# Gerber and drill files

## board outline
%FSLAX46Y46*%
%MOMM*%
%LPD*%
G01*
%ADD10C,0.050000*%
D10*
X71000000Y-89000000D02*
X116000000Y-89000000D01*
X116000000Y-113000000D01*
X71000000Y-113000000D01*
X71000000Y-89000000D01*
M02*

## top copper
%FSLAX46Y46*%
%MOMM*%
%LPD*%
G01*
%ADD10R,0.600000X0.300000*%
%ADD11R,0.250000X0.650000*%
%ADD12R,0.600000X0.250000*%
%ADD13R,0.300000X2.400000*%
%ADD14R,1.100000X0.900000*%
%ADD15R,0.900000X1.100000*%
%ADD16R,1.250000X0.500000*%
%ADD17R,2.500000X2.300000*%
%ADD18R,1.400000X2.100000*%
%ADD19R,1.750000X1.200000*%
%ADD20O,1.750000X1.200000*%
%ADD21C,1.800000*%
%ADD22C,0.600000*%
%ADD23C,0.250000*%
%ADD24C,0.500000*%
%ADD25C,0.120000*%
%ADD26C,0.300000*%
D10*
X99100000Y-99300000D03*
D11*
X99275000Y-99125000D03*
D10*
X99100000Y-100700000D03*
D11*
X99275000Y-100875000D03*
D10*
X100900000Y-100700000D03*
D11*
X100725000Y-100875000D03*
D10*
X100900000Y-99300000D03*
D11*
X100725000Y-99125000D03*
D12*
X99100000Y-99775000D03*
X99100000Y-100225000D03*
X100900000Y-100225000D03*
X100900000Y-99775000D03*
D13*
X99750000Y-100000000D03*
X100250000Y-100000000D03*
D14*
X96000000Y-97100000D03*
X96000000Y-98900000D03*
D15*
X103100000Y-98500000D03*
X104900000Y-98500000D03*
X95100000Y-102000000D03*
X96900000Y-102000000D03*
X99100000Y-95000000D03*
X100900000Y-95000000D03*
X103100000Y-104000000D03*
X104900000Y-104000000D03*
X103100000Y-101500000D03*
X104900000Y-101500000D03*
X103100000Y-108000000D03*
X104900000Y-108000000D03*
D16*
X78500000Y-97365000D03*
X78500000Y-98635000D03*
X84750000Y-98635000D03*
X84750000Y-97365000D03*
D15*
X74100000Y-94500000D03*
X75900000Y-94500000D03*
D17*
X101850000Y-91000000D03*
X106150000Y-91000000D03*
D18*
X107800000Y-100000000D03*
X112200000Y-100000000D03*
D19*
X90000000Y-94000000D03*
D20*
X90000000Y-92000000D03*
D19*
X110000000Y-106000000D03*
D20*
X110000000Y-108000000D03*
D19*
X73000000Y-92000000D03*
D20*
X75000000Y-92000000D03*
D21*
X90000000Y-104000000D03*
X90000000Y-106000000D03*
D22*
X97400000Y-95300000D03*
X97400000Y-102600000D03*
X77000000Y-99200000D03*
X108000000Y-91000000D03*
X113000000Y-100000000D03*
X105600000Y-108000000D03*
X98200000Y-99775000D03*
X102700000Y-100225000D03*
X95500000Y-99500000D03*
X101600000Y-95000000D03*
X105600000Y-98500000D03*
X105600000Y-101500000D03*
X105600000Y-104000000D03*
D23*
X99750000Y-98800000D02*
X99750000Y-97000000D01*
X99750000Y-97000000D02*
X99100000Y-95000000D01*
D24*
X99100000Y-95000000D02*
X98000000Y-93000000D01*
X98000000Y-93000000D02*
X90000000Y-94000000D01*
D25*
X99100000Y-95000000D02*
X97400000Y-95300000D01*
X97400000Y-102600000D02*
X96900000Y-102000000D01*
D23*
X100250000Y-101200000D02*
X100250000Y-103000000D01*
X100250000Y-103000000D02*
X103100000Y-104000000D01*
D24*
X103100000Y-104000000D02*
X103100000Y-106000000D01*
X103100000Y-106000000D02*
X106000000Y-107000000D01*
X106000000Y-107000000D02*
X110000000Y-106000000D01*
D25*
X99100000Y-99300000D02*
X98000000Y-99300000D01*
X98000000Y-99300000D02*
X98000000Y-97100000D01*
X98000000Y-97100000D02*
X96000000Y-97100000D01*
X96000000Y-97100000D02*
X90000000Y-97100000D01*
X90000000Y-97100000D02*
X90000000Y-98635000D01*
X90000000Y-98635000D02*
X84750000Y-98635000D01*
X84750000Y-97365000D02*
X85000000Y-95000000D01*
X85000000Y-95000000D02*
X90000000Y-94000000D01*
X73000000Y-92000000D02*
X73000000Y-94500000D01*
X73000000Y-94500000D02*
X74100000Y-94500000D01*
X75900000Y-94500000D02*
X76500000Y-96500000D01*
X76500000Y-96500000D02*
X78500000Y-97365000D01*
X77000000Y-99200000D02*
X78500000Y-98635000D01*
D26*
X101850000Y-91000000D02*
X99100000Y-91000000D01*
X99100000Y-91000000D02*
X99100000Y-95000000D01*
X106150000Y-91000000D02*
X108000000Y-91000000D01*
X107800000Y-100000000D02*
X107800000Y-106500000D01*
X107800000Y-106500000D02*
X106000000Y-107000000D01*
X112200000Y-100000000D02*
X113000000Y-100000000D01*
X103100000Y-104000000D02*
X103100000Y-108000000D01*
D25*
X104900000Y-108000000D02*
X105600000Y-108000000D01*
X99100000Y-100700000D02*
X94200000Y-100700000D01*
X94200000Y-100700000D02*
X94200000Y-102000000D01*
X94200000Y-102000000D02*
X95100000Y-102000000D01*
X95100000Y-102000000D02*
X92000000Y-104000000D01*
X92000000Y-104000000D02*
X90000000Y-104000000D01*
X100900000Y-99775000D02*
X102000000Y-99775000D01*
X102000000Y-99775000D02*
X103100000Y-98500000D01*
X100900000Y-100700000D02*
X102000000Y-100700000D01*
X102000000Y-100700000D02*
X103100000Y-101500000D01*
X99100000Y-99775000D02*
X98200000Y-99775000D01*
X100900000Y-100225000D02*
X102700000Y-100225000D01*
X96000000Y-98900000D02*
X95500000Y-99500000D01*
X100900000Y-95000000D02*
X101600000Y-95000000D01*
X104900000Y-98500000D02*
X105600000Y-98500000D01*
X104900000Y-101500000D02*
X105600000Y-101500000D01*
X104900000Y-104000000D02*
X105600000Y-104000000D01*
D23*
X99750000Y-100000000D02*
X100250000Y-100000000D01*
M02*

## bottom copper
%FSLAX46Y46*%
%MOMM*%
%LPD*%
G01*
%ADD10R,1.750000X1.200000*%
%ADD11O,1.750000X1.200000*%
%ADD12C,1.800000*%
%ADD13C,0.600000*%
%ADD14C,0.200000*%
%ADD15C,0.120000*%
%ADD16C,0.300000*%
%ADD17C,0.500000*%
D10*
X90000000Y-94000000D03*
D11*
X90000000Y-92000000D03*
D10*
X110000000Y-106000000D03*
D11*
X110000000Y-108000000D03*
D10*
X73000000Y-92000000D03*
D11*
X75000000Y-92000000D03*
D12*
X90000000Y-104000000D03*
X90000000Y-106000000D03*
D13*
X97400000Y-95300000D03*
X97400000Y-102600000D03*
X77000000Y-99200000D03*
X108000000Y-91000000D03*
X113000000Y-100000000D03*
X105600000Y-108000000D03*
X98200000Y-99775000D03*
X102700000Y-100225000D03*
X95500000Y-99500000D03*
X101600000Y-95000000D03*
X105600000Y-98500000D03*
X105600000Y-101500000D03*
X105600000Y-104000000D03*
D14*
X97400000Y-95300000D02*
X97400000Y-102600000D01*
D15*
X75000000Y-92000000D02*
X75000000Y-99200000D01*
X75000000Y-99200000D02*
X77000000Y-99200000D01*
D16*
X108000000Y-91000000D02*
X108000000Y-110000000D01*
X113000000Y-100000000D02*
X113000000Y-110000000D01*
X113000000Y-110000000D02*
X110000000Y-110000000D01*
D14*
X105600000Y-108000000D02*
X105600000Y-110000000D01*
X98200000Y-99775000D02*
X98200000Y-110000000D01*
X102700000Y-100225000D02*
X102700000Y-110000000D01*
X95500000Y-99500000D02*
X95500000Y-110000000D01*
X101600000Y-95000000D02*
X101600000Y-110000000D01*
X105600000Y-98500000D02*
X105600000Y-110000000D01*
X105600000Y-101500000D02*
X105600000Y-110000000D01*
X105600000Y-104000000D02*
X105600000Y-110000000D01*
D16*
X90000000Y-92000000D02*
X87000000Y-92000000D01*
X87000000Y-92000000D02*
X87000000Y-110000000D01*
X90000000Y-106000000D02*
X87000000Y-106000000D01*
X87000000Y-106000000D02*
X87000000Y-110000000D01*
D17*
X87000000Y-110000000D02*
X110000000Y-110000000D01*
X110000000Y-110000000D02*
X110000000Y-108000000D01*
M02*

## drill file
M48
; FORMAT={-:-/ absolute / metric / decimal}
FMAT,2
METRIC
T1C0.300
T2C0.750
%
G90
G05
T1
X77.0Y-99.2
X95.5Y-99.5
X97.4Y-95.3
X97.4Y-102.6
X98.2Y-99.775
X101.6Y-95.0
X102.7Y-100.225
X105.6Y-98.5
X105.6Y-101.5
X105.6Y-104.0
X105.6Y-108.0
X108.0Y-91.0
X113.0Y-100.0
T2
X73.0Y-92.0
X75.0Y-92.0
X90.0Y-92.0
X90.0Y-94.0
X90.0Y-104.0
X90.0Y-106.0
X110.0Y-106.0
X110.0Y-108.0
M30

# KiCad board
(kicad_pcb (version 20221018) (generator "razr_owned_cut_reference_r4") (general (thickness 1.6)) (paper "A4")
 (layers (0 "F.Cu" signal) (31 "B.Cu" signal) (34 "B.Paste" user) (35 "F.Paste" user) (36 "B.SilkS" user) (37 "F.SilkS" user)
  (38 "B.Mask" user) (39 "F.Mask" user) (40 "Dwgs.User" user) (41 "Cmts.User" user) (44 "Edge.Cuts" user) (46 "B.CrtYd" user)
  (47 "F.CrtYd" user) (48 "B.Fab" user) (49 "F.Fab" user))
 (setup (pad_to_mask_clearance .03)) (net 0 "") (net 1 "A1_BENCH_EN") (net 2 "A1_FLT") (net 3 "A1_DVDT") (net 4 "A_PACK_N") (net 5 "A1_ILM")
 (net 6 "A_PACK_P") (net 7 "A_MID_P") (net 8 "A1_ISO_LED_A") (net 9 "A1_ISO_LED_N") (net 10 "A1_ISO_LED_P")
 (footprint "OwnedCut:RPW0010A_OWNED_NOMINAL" (layer "F.Cu") (at 100 100)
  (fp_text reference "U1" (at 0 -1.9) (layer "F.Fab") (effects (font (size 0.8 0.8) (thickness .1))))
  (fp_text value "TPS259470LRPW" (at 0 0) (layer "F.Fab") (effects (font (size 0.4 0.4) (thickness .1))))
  (pad "1" smd rect (at -0.9 -0.7) (size 0.6 0.3) (layers "F.Cu" "F.Paste" "F.Mask") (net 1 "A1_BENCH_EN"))
  (pad "1" smd rect (at -0.725 -0.875) (size 0.25 0.65) (layers "F.Cu" "F.Paste" "F.Mask") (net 1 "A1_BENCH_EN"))
  (pad "4" smd rect (at -0.9 0.7) (size 0.6 0.3) (layers "F.Cu" "F.Paste" "F.Mask") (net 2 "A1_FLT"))
  (pad "4" smd rect (at -0.725 0.875) (size 0.25 0.65) (layers "F.Cu" "F.Paste" "F.Mask") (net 2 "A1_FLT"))
  (pad "7" smd rect (at 0.9 0.7) (size 0.6 0.3) (layers "F.Cu" "F.Paste" "F.Mask") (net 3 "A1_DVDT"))
  (pad "7" smd rect (at 0.725 0.875) (size 0.25 0.65) (layers "F.Cu" "F.Paste" "F.Mask") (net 3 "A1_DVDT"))
  (pad "10" smd rect (at 0.9 -0.7) (size 0.6 0.3) (layers "F.Cu" "F.Paste" "F.Mask"))
  (pad "10" smd rect (at 0.725 -0.875) (size 0.25 0.65) (layers "F.Cu" "F.Paste" "F.Mask"))
  (pad "2" smd rect (at -0.9 -0.225) (size 0.6 0.25) (layers "F.Cu" "F.Paste" "F.Mask") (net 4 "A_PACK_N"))
  (pad "3" smd rect (at -0.9 0.225) (size 0.6 0.25) (layers "F.Cu" "F.Paste" "F.Mask"))
  (pad "8" smd rect (at 0.9 0.225) (size 0.6 0.25) (layers "F.Cu" "F.Paste" "F.Mask") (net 4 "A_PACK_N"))
  (pad "9" smd rect (at 0.9 -0.225) (size 0.6 0.25) (layers "F.Cu" "F.Paste" "F.Mask") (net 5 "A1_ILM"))
  (pad "5" smd rect (at -0.25 0) (size 0.3 2.4) (layers "F.Cu" "F.Paste" "F.Mask") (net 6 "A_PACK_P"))
  (pad "6" smd rect (at 0.25 0) (size 0.3 2.4) (layers "F.Cu" "F.Paste" "F.Mask") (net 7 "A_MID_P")))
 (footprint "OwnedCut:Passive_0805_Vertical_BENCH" (layer "F.Cu") (at 96 98)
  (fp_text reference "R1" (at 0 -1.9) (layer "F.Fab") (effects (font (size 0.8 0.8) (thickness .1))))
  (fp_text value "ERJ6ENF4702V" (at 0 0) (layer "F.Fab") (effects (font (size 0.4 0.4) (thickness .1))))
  (pad "1" smd rect (at 0 -0.9) (size 1.1 0.9) (layers "F.Cu" "F.Paste" "F.Mask") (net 1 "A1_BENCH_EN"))
  (pad "2" smd rect (at 0 0.9) (size 1.1 0.9) (layers "F.Cu" "F.Paste" "F.Mask") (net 4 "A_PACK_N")))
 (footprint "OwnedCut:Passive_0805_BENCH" (layer "F.Cu") (at 104 98.5)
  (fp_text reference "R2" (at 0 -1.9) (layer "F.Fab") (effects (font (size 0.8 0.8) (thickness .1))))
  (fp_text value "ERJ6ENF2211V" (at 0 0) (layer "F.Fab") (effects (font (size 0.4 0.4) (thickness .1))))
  (pad "1" smd rect (at -0.9 0) (size 0.9 1.1) (layers "F.Cu" "F.Paste" "F.Mask") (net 5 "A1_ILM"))
  (pad "2" smd rect (at 0.9 0) (size 0.9 1.1) (layers "F.Cu" "F.Paste" "F.Mask") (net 4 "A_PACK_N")))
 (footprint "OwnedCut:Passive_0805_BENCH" (layer "F.Cu") (at 96 102)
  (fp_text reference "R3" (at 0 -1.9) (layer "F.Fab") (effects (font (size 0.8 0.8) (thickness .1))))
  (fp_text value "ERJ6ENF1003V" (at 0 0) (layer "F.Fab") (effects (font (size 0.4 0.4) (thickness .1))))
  (pad "1" smd rect (at -0.9 0) (size 0.9 1.1) (layers "F.Cu" "F.Paste" "F.Mask") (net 2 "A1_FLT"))
  (pad "2" smd rect (at 0.9 0) (size 0.9 1.1) (layers "F.Cu" "F.Paste" "F.Mask") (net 6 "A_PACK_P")))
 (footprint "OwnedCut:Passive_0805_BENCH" (layer "F.Cu") (at 100 95)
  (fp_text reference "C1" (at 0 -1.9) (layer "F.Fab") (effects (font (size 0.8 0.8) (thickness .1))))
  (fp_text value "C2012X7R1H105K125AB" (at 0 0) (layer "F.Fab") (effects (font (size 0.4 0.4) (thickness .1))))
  (pad "1" smd rect (at -0.9 0) (size 0.9 1.1) (layers "F.Cu" "F.Paste" "F.Mask") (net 6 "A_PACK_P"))
  (pad "2" smd rect (at 0.9 0) (size 0.9 1.1) (layers "F.Cu" "F.Paste" "F.Mask") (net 4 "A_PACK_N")))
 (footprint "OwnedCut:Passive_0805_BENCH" (layer "F.Cu") (at 104 104)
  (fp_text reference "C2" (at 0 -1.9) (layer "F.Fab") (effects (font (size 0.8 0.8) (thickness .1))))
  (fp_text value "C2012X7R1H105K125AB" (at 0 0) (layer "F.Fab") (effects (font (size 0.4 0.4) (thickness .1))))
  (pad "1" smd rect (at -0.9 0) (size 0.9 1.1) (layers "F.Cu" "F.Paste" "F.Mask") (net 7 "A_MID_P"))
  (pad "2" smd rect (at 0.9 0) (size 0.9 1.1) (layers "F.Cu" "F.Paste" "F.Mask") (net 4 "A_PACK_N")))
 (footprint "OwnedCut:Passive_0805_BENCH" (layer "F.Cu") (at 104 101.5)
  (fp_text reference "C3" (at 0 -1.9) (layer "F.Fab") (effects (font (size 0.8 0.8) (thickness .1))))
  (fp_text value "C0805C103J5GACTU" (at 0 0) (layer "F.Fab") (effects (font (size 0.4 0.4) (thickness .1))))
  (pad "1" smd rect (at -0.9 0) (size 0.9 1.1) (layers "F.Cu" "F.Paste" "F.Mask") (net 3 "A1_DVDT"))
  (pad "2" smd rect (at 0.9 0) (size 0.9 1.1) (layers "F.Cu" "F.Paste" "F.Mask") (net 4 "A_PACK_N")))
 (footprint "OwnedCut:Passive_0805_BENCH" (layer "F.Cu") (at 104 108)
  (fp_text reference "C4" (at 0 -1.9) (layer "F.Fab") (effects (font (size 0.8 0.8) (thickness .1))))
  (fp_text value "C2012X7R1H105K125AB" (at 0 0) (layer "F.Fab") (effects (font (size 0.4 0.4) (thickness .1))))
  (pad "1" smd rect (at -0.9 0) (size 0.9 1.1) (layers "F.Cu" "F.Paste" "F.Mask") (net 7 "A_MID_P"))
  (pad "2" smd rect (at 0.9 0) (size 0.9 1.1) (layers "F.Cu" "F.Paste" "F.Mask") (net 4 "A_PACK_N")))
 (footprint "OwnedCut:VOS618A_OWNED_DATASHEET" (layer "F.Cu") (at 81.625 98)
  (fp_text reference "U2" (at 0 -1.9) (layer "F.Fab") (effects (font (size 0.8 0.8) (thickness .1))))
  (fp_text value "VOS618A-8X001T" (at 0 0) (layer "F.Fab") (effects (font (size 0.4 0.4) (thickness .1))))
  (pad "1" smd rect (at -3.125 -0.635) (size 1.25 0.5) (layers "F.Cu" "F.Paste" "F.Mask") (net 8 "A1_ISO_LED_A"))
  (pad "2" smd rect (at -3.125 0.635) (size 1.25 0.5) (layers "F.Cu" "F.Paste" "F.Mask") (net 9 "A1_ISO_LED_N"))
  (pad "3" smd rect (at 3.125 0.635) (size 1.25 0.5) (layers "F.Cu" "F.Paste" "F.Mask") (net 1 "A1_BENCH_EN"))
  (pad "4" smd rect (at 3.125 -0.635) (size 1.25 0.5) (layers "F.Cu" "F.Paste" "F.Mask") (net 6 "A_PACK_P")))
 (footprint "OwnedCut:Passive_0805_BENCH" (layer "F.Cu") (at 75 94.5)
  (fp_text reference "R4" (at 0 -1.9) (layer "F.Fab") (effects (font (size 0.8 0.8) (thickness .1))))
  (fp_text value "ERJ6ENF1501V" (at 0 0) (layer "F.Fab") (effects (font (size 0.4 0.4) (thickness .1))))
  (pad "1" smd rect (at -0.9 0) (size 0.9 1.1) (layers "F.Cu" "F.Paste" "F.Mask") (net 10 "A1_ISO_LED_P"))
  (pad "2" smd rect (at 0.9 0) (size 0.9 1.1) (layers "F.Cu" "F.Paste" "F.Mask") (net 8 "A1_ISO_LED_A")))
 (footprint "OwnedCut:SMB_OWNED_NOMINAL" (layer "F.Cu") (at 104 91)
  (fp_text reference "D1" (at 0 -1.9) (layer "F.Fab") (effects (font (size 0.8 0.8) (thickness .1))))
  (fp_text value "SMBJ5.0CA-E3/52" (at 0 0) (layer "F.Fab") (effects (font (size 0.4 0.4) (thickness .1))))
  (pad "1" smd rect (at -2.15 0) (size 2.5 2.3) (layers "F.Cu" "F.Paste" "F.Mask") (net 6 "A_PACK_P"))
  (pad "2" smd rect (at 2.15 0) (size 2.5 2.3) (layers "F.Cu" "F.Paste" "F.Mask") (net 4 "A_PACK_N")))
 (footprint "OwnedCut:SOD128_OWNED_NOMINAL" (layer "F.Cu") (at 110 100)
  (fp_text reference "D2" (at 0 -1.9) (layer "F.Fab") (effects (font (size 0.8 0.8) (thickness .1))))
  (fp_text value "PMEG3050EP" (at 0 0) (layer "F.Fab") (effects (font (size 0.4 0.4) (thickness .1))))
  (pad "1" smd rect (at -2.2 0) (size 1.4 2.1) (layers "F.Cu" "F.Paste" "F.Mask") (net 7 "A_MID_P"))
  (pad "2" smd rect (at 2.2 0) (size 1.4 2.1) (layers "F.Cu" "F.Paste" "F.Mask") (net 4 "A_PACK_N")))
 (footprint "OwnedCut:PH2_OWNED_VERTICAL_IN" (layer "F.Cu") (at 90 94)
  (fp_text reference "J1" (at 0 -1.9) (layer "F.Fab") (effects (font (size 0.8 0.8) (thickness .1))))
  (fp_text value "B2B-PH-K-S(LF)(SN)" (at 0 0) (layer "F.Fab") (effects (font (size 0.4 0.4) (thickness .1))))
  (pad "1" thru_hole rect (at 0 0) (size 1.75 1.2) (drill .75) (layers "*.Cu" "*.Mask") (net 6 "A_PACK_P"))
  (pad "2" thru_hole oval (at 0 -2) (size 1.75 1.2) (drill .75) (layers "*.Cu" "*.Mask") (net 4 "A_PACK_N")))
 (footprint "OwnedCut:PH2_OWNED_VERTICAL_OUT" (layer "F.Cu") (at 110 106)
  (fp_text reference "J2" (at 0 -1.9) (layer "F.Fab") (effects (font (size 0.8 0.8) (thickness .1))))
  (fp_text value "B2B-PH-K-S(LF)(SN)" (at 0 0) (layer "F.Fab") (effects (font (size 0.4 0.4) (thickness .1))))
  (pad "1" thru_hole rect (at 0 0) (size 1.75 1.2) (drill .75) (layers "*.Cu" "*.Mask") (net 7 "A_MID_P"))
  (pad "2" thru_hole oval (at 0 2) (size 1.75 1.2) (drill .75) (layers "*.Cu" "*.Mask") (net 4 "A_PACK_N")))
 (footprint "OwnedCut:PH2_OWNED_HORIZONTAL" (layer "F.Cu") (at 73 92)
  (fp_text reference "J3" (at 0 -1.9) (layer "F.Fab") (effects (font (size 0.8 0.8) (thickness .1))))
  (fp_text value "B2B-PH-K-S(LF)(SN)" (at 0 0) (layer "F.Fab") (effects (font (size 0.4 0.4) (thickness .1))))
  (pad "1" thru_hole rect (at 0 0) (size 1.75 1.2) (drill .75) (layers "*.Cu" "*.Mask") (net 10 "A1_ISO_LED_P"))
  (pad "2" thru_hole oval (at 2 0) (size 1.75 1.2) (drill .75) (layers "*.Cu" "*.Mask") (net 9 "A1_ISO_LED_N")))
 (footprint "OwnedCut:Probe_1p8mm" (layer "F.Cu") (at 90 104)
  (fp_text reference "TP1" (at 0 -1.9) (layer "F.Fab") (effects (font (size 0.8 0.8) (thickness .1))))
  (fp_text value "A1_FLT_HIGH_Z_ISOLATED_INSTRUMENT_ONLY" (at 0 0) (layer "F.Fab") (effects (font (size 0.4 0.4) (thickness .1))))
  (pad "1" thru_hole circle (at 0 0) (size 1.8 1.8) (drill .75) (layers "*.Cu" "*.Mask") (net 2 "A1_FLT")))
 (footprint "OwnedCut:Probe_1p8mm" (layer "F.Cu") (at 90 106)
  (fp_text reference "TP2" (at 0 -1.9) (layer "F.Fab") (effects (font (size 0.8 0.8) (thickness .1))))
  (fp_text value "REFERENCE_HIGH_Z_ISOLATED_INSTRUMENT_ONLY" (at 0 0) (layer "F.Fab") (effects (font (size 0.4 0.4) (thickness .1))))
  (pad "1" thru_hole circle (at 0 0) (size 1.8 1.8) (drill .75) (layers "*.Cu" "*.Mask") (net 4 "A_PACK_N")))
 (segment (start 99.75 98.8) (end 99.75 97) (width 0.25) (layer "F.Cu") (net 6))
 (segment (start 99.75 97) (end 99.1 95) (width 0.25) (layer "F.Cu") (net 6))
 (segment (start 99.1 95) (end 98 93) (width 0.5) (layer "F.Cu") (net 6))
 (segment (start 98 93) (end 90 94) (width 0.5) (layer "F.Cu") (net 6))
 (segment (start 99.1 95) (end 97.4 95.3) (width 0.12) (layer "F.Cu") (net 6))
 (via (at 97.4 95.3) (size .6) (drill .3) (layers "F.Cu" "B.Cu") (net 6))
 (segment (start 97.4 95.3) (end 97.4 102.6) (width 0.2) (layer "B.Cu") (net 6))
 (via (at 97.4 102.6) (size .6) (drill .3) (layers "F.Cu" "B.Cu") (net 6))
 (segment (start 97.4 102.6) (end 96.9 102) (width 0.12) (layer "F.Cu") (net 6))
 (segment (start 100.25 101.2) (end 100.25 103) (width 0.25) (layer "F.Cu") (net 7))
 (segment (start 100.25 103) (end 103.1 104) (width 0.25) (layer "F.Cu") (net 7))
 (segment (start 103.1 104) (end 103.1 106) (width 0.5) (layer "F.Cu") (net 7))
 (segment (start 103.1 106) (end 106 107) (width 0.5) (layer "F.Cu") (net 7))
 (segment (start 106 107) (end 110 106) (width 0.5) (layer "F.Cu") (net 7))
 (segment (start 99.1 99.3) (end 98 99.3) (width 0.12) (layer "F.Cu") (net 1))
 (segment (start 98 99.3) (end 98 97.1) (width 0.12) (layer "F.Cu") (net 1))
 (segment (start 98 97.1) (end 96 97.1) (width 0.12) (layer "F.Cu") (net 1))
 (segment (start 96 97.1) (end 90 97.1) (width 0.12) (layer "F.Cu") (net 1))
 (segment (start 90 97.1) (end 90 98.635) (width 0.12) (layer "F.Cu") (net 1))
 (segment (start 90 98.635) (end 84.75 98.635) (width 0.12) (layer "F.Cu") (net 1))
 (segment (start 84.75 97.365) (end 85 95) (width 0.12) (layer "F.Cu") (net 6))
 (segment (start 85 95) (end 90 94) (width 0.12) (layer "F.Cu") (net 6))
 (segment (start 73 92) (end 73 94.5) (width 0.12) (layer "F.Cu") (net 10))
 (segment (start 73 94.5) (end 74.1 94.5) (width 0.12) (layer "F.Cu") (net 10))
 (segment (start 75.9 94.5) (end 76.5 96.5) (width 0.12) (layer "F.Cu") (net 8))
 (segment (start 76.5 96.5) (end 78.5 97.365) (width 0.12) (layer "F.Cu") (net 8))
 (segment (start 75 92) (end 75 99.2) (width 0.12) (layer "B.Cu") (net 9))
 (segment (start 75 99.2) (end 77 99.2) (width 0.12) (layer "B.Cu") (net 9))
 (via (at 77 99.2) (size .6) (drill .3) (layers "F.Cu" "B.Cu") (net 9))
 (segment (start 77 99.2) (end 78.5 98.635) (width 0.12) (layer "F.Cu") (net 9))
 (segment (start 101.85 91) (end 99.1 91) (width 0.3) (layer "F.Cu") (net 6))
 (segment (start 99.1 91) (end 99.1 95) (width 0.3) (layer "F.Cu") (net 6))
 (segment (start 106.15 91) (end 108 91) (width 0.3) (layer "F.Cu") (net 4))
 (via (at 108 91) (size .6) (drill .3) (layers "F.Cu" "B.Cu") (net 4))
 (segment (start 108 91) (end 108 110) (width 0.3) (layer "B.Cu") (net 4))
 (segment (start 107.8 100) (end 107.8 106.5) (width 0.3) (layer "F.Cu") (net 7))
 (segment (start 107.8 106.5) (end 106 107) (width 0.3) (layer "F.Cu") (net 7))
 (segment (start 112.2 100) (end 113 100) (width 0.3) (layer "F.Cu") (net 4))
 (via (at 113 100) (size .6) (drill .3) (layers "F.Cu" "B.Cu") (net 4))
 (segment (start 113 100) (end 113 110) (width 0.3) (layer "B.Cu") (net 4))
 (segment (start 113 110) (end 110 110) (width 0.3) (layer "B.Cu") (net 4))
 (segment (start 103.1 104) (end 103.1 108) (width 0.3) (layer "F.Cu") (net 7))
 (segment (start 104.9 108) (end 105.6 108) (width 0.12) (layer "F.Cu") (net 4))
 (via (at 105.6 108) (size .6) (drill .3) (layers "F.Cu" "B.Cu") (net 4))
 (segment (start 105.6 108) (end 105.6 110) (width 0.2) (layer "B.Cu") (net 4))
 (segment (start 99.1 100.7) (end 94.2 100.7) (width 0.12) (layer "F.Cu") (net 2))
 (segment (start 94.2 100.7) (end 94.2 102) (width 0.12) (layer "F.Cu") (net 2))
 (segment (start 94.2 102) (end 95.1 102) (width 0.12) (layer "F.Cu") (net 2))
 (segment (start 95.1 102) (end 92 104) (width 0.12) (layer "F.Cu") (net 2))
 (segment (start 92 104) (end 90 104) (width 0.12) (layer "F.Cu") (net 2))
 (segment (start 100.9 99.775) (end 102 99.775) (width 0.12) (layer "F.Cu") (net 5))
 (segment (start 102 99.775) (end 103.1 98.5) (width 0.12) (layer "F.Cu") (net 5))
 (segment (start 100.9 100.7) (end 102 100.7) (width 0.12) (layer "F.Cu") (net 3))
 (segment (start 102 100.7) (end 103.1 101.5) (width 0.12) (layer "F.Cu") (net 3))
 (segment (start 99.1 99.775) (end 98.2 99.775) (width 0.12) (layer "F.Cu") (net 4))
 (via (at 98.2 99.775) (size .6) (drill .3) (layers "F.Cu" "B.Cu") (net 4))
 (segment (start 98.2 99.775) (end 98.2 110) (width 0.2) (layer "B.Cu") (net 4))
 (segment (start 100.9 100.225) (end 102.7 100.225) (width 0.12) (layer "F.Cu") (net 4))
 (via (at 102.7 100.225) (size .6) (drill .3) (layers "F.Cu" "B.Cu") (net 4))
 (segment (start 102.7 100.225) (end 102.7 110) (width 0.2) (layer "B.Cu") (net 4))
 (segment (start 96 98.9) (end 95.5 99.5) (width 0.12) (layer "F.Cu") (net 4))
 (via (at 95.5 99.5) (size .6) (drill .3) (layers "F.Cu" "B.Cu") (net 4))
 (segment (start 95.5 99.5) (end 95.5 110) (width 0.2) (layer "B.Cu") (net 4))
 (segment (start 100.9 95) (end 101.6 95) (width 0.12) (layer "F.Cu") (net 4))
 (via (at 101.6 95) (size .6) (drill .3) (layers "F.Cu" "B.Cu") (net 4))
 (segment (start 101.6 95) (end 101.6 110) (width 0.2) (layer "B.Cu") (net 4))
 (segment (start 104.9 98.5) (end 105.6 98.5) (width 0.12) (layer "F.Cu") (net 4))
 (via (at 105.6 98.5) (size .6) (drill .3) (layers "F.Cu" "B.Cu") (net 4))
 (segment (start 105.6 98.5) (end 105.6 110) (width 0.2) (layer "B.Cu") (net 4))
 (segment (start 104.9 101.5) (end 105.6 101.5) (width 0.12) (layer "F.Cu") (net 4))
 (via (at 105.6 101.5) (size .6) (drill .3) (layers "F.Cu" "B.Cu") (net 4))
 (segment (start 105.6 101.5) (end 105.6 110) (width 0.2) (layer "B.Cu") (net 4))
 (segment (start 104.9 104) (end 105.6 104) (width 0.12) (layer "F.Cu") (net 4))
 (via (at 105.6 104) (size .6) (drill .3) (layers "F.Cu" "B.Cu") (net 4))
 (segment (start 105.6 104) (end 105.6 110) (width 0.2) (layer "B.Cu") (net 4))
 (segment (start 90 92) (end 87 92) (width 0.3) (layer "B.Cu") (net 4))
 (segment (start 87 92) (end 87 110) (width 0.3) (layer "B.Cu") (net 4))
 (segment (start 90 106) (end 87 106) (width 0.3) (layer "B.Cu") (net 4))
 (segment (start 87 106) (end 87 110) (width 0.3) (layer "B.Cu") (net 4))
 (segment (start 87 110) (end 110 110) (width 0.5) (layer "B.Cu") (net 4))
 (segment (start 110 110) (end 110 108) (width 0.5) (layer "B.Cu") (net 4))
 (gr_rect (start 71 89) (end 116 113) (stroke (width .05) (type default)) (fill none) (layer "Edge.Cuts"))
 (segment (start 99.75 100) (end 100.25 100) (width .25) (layer "F.Cu") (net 6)))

